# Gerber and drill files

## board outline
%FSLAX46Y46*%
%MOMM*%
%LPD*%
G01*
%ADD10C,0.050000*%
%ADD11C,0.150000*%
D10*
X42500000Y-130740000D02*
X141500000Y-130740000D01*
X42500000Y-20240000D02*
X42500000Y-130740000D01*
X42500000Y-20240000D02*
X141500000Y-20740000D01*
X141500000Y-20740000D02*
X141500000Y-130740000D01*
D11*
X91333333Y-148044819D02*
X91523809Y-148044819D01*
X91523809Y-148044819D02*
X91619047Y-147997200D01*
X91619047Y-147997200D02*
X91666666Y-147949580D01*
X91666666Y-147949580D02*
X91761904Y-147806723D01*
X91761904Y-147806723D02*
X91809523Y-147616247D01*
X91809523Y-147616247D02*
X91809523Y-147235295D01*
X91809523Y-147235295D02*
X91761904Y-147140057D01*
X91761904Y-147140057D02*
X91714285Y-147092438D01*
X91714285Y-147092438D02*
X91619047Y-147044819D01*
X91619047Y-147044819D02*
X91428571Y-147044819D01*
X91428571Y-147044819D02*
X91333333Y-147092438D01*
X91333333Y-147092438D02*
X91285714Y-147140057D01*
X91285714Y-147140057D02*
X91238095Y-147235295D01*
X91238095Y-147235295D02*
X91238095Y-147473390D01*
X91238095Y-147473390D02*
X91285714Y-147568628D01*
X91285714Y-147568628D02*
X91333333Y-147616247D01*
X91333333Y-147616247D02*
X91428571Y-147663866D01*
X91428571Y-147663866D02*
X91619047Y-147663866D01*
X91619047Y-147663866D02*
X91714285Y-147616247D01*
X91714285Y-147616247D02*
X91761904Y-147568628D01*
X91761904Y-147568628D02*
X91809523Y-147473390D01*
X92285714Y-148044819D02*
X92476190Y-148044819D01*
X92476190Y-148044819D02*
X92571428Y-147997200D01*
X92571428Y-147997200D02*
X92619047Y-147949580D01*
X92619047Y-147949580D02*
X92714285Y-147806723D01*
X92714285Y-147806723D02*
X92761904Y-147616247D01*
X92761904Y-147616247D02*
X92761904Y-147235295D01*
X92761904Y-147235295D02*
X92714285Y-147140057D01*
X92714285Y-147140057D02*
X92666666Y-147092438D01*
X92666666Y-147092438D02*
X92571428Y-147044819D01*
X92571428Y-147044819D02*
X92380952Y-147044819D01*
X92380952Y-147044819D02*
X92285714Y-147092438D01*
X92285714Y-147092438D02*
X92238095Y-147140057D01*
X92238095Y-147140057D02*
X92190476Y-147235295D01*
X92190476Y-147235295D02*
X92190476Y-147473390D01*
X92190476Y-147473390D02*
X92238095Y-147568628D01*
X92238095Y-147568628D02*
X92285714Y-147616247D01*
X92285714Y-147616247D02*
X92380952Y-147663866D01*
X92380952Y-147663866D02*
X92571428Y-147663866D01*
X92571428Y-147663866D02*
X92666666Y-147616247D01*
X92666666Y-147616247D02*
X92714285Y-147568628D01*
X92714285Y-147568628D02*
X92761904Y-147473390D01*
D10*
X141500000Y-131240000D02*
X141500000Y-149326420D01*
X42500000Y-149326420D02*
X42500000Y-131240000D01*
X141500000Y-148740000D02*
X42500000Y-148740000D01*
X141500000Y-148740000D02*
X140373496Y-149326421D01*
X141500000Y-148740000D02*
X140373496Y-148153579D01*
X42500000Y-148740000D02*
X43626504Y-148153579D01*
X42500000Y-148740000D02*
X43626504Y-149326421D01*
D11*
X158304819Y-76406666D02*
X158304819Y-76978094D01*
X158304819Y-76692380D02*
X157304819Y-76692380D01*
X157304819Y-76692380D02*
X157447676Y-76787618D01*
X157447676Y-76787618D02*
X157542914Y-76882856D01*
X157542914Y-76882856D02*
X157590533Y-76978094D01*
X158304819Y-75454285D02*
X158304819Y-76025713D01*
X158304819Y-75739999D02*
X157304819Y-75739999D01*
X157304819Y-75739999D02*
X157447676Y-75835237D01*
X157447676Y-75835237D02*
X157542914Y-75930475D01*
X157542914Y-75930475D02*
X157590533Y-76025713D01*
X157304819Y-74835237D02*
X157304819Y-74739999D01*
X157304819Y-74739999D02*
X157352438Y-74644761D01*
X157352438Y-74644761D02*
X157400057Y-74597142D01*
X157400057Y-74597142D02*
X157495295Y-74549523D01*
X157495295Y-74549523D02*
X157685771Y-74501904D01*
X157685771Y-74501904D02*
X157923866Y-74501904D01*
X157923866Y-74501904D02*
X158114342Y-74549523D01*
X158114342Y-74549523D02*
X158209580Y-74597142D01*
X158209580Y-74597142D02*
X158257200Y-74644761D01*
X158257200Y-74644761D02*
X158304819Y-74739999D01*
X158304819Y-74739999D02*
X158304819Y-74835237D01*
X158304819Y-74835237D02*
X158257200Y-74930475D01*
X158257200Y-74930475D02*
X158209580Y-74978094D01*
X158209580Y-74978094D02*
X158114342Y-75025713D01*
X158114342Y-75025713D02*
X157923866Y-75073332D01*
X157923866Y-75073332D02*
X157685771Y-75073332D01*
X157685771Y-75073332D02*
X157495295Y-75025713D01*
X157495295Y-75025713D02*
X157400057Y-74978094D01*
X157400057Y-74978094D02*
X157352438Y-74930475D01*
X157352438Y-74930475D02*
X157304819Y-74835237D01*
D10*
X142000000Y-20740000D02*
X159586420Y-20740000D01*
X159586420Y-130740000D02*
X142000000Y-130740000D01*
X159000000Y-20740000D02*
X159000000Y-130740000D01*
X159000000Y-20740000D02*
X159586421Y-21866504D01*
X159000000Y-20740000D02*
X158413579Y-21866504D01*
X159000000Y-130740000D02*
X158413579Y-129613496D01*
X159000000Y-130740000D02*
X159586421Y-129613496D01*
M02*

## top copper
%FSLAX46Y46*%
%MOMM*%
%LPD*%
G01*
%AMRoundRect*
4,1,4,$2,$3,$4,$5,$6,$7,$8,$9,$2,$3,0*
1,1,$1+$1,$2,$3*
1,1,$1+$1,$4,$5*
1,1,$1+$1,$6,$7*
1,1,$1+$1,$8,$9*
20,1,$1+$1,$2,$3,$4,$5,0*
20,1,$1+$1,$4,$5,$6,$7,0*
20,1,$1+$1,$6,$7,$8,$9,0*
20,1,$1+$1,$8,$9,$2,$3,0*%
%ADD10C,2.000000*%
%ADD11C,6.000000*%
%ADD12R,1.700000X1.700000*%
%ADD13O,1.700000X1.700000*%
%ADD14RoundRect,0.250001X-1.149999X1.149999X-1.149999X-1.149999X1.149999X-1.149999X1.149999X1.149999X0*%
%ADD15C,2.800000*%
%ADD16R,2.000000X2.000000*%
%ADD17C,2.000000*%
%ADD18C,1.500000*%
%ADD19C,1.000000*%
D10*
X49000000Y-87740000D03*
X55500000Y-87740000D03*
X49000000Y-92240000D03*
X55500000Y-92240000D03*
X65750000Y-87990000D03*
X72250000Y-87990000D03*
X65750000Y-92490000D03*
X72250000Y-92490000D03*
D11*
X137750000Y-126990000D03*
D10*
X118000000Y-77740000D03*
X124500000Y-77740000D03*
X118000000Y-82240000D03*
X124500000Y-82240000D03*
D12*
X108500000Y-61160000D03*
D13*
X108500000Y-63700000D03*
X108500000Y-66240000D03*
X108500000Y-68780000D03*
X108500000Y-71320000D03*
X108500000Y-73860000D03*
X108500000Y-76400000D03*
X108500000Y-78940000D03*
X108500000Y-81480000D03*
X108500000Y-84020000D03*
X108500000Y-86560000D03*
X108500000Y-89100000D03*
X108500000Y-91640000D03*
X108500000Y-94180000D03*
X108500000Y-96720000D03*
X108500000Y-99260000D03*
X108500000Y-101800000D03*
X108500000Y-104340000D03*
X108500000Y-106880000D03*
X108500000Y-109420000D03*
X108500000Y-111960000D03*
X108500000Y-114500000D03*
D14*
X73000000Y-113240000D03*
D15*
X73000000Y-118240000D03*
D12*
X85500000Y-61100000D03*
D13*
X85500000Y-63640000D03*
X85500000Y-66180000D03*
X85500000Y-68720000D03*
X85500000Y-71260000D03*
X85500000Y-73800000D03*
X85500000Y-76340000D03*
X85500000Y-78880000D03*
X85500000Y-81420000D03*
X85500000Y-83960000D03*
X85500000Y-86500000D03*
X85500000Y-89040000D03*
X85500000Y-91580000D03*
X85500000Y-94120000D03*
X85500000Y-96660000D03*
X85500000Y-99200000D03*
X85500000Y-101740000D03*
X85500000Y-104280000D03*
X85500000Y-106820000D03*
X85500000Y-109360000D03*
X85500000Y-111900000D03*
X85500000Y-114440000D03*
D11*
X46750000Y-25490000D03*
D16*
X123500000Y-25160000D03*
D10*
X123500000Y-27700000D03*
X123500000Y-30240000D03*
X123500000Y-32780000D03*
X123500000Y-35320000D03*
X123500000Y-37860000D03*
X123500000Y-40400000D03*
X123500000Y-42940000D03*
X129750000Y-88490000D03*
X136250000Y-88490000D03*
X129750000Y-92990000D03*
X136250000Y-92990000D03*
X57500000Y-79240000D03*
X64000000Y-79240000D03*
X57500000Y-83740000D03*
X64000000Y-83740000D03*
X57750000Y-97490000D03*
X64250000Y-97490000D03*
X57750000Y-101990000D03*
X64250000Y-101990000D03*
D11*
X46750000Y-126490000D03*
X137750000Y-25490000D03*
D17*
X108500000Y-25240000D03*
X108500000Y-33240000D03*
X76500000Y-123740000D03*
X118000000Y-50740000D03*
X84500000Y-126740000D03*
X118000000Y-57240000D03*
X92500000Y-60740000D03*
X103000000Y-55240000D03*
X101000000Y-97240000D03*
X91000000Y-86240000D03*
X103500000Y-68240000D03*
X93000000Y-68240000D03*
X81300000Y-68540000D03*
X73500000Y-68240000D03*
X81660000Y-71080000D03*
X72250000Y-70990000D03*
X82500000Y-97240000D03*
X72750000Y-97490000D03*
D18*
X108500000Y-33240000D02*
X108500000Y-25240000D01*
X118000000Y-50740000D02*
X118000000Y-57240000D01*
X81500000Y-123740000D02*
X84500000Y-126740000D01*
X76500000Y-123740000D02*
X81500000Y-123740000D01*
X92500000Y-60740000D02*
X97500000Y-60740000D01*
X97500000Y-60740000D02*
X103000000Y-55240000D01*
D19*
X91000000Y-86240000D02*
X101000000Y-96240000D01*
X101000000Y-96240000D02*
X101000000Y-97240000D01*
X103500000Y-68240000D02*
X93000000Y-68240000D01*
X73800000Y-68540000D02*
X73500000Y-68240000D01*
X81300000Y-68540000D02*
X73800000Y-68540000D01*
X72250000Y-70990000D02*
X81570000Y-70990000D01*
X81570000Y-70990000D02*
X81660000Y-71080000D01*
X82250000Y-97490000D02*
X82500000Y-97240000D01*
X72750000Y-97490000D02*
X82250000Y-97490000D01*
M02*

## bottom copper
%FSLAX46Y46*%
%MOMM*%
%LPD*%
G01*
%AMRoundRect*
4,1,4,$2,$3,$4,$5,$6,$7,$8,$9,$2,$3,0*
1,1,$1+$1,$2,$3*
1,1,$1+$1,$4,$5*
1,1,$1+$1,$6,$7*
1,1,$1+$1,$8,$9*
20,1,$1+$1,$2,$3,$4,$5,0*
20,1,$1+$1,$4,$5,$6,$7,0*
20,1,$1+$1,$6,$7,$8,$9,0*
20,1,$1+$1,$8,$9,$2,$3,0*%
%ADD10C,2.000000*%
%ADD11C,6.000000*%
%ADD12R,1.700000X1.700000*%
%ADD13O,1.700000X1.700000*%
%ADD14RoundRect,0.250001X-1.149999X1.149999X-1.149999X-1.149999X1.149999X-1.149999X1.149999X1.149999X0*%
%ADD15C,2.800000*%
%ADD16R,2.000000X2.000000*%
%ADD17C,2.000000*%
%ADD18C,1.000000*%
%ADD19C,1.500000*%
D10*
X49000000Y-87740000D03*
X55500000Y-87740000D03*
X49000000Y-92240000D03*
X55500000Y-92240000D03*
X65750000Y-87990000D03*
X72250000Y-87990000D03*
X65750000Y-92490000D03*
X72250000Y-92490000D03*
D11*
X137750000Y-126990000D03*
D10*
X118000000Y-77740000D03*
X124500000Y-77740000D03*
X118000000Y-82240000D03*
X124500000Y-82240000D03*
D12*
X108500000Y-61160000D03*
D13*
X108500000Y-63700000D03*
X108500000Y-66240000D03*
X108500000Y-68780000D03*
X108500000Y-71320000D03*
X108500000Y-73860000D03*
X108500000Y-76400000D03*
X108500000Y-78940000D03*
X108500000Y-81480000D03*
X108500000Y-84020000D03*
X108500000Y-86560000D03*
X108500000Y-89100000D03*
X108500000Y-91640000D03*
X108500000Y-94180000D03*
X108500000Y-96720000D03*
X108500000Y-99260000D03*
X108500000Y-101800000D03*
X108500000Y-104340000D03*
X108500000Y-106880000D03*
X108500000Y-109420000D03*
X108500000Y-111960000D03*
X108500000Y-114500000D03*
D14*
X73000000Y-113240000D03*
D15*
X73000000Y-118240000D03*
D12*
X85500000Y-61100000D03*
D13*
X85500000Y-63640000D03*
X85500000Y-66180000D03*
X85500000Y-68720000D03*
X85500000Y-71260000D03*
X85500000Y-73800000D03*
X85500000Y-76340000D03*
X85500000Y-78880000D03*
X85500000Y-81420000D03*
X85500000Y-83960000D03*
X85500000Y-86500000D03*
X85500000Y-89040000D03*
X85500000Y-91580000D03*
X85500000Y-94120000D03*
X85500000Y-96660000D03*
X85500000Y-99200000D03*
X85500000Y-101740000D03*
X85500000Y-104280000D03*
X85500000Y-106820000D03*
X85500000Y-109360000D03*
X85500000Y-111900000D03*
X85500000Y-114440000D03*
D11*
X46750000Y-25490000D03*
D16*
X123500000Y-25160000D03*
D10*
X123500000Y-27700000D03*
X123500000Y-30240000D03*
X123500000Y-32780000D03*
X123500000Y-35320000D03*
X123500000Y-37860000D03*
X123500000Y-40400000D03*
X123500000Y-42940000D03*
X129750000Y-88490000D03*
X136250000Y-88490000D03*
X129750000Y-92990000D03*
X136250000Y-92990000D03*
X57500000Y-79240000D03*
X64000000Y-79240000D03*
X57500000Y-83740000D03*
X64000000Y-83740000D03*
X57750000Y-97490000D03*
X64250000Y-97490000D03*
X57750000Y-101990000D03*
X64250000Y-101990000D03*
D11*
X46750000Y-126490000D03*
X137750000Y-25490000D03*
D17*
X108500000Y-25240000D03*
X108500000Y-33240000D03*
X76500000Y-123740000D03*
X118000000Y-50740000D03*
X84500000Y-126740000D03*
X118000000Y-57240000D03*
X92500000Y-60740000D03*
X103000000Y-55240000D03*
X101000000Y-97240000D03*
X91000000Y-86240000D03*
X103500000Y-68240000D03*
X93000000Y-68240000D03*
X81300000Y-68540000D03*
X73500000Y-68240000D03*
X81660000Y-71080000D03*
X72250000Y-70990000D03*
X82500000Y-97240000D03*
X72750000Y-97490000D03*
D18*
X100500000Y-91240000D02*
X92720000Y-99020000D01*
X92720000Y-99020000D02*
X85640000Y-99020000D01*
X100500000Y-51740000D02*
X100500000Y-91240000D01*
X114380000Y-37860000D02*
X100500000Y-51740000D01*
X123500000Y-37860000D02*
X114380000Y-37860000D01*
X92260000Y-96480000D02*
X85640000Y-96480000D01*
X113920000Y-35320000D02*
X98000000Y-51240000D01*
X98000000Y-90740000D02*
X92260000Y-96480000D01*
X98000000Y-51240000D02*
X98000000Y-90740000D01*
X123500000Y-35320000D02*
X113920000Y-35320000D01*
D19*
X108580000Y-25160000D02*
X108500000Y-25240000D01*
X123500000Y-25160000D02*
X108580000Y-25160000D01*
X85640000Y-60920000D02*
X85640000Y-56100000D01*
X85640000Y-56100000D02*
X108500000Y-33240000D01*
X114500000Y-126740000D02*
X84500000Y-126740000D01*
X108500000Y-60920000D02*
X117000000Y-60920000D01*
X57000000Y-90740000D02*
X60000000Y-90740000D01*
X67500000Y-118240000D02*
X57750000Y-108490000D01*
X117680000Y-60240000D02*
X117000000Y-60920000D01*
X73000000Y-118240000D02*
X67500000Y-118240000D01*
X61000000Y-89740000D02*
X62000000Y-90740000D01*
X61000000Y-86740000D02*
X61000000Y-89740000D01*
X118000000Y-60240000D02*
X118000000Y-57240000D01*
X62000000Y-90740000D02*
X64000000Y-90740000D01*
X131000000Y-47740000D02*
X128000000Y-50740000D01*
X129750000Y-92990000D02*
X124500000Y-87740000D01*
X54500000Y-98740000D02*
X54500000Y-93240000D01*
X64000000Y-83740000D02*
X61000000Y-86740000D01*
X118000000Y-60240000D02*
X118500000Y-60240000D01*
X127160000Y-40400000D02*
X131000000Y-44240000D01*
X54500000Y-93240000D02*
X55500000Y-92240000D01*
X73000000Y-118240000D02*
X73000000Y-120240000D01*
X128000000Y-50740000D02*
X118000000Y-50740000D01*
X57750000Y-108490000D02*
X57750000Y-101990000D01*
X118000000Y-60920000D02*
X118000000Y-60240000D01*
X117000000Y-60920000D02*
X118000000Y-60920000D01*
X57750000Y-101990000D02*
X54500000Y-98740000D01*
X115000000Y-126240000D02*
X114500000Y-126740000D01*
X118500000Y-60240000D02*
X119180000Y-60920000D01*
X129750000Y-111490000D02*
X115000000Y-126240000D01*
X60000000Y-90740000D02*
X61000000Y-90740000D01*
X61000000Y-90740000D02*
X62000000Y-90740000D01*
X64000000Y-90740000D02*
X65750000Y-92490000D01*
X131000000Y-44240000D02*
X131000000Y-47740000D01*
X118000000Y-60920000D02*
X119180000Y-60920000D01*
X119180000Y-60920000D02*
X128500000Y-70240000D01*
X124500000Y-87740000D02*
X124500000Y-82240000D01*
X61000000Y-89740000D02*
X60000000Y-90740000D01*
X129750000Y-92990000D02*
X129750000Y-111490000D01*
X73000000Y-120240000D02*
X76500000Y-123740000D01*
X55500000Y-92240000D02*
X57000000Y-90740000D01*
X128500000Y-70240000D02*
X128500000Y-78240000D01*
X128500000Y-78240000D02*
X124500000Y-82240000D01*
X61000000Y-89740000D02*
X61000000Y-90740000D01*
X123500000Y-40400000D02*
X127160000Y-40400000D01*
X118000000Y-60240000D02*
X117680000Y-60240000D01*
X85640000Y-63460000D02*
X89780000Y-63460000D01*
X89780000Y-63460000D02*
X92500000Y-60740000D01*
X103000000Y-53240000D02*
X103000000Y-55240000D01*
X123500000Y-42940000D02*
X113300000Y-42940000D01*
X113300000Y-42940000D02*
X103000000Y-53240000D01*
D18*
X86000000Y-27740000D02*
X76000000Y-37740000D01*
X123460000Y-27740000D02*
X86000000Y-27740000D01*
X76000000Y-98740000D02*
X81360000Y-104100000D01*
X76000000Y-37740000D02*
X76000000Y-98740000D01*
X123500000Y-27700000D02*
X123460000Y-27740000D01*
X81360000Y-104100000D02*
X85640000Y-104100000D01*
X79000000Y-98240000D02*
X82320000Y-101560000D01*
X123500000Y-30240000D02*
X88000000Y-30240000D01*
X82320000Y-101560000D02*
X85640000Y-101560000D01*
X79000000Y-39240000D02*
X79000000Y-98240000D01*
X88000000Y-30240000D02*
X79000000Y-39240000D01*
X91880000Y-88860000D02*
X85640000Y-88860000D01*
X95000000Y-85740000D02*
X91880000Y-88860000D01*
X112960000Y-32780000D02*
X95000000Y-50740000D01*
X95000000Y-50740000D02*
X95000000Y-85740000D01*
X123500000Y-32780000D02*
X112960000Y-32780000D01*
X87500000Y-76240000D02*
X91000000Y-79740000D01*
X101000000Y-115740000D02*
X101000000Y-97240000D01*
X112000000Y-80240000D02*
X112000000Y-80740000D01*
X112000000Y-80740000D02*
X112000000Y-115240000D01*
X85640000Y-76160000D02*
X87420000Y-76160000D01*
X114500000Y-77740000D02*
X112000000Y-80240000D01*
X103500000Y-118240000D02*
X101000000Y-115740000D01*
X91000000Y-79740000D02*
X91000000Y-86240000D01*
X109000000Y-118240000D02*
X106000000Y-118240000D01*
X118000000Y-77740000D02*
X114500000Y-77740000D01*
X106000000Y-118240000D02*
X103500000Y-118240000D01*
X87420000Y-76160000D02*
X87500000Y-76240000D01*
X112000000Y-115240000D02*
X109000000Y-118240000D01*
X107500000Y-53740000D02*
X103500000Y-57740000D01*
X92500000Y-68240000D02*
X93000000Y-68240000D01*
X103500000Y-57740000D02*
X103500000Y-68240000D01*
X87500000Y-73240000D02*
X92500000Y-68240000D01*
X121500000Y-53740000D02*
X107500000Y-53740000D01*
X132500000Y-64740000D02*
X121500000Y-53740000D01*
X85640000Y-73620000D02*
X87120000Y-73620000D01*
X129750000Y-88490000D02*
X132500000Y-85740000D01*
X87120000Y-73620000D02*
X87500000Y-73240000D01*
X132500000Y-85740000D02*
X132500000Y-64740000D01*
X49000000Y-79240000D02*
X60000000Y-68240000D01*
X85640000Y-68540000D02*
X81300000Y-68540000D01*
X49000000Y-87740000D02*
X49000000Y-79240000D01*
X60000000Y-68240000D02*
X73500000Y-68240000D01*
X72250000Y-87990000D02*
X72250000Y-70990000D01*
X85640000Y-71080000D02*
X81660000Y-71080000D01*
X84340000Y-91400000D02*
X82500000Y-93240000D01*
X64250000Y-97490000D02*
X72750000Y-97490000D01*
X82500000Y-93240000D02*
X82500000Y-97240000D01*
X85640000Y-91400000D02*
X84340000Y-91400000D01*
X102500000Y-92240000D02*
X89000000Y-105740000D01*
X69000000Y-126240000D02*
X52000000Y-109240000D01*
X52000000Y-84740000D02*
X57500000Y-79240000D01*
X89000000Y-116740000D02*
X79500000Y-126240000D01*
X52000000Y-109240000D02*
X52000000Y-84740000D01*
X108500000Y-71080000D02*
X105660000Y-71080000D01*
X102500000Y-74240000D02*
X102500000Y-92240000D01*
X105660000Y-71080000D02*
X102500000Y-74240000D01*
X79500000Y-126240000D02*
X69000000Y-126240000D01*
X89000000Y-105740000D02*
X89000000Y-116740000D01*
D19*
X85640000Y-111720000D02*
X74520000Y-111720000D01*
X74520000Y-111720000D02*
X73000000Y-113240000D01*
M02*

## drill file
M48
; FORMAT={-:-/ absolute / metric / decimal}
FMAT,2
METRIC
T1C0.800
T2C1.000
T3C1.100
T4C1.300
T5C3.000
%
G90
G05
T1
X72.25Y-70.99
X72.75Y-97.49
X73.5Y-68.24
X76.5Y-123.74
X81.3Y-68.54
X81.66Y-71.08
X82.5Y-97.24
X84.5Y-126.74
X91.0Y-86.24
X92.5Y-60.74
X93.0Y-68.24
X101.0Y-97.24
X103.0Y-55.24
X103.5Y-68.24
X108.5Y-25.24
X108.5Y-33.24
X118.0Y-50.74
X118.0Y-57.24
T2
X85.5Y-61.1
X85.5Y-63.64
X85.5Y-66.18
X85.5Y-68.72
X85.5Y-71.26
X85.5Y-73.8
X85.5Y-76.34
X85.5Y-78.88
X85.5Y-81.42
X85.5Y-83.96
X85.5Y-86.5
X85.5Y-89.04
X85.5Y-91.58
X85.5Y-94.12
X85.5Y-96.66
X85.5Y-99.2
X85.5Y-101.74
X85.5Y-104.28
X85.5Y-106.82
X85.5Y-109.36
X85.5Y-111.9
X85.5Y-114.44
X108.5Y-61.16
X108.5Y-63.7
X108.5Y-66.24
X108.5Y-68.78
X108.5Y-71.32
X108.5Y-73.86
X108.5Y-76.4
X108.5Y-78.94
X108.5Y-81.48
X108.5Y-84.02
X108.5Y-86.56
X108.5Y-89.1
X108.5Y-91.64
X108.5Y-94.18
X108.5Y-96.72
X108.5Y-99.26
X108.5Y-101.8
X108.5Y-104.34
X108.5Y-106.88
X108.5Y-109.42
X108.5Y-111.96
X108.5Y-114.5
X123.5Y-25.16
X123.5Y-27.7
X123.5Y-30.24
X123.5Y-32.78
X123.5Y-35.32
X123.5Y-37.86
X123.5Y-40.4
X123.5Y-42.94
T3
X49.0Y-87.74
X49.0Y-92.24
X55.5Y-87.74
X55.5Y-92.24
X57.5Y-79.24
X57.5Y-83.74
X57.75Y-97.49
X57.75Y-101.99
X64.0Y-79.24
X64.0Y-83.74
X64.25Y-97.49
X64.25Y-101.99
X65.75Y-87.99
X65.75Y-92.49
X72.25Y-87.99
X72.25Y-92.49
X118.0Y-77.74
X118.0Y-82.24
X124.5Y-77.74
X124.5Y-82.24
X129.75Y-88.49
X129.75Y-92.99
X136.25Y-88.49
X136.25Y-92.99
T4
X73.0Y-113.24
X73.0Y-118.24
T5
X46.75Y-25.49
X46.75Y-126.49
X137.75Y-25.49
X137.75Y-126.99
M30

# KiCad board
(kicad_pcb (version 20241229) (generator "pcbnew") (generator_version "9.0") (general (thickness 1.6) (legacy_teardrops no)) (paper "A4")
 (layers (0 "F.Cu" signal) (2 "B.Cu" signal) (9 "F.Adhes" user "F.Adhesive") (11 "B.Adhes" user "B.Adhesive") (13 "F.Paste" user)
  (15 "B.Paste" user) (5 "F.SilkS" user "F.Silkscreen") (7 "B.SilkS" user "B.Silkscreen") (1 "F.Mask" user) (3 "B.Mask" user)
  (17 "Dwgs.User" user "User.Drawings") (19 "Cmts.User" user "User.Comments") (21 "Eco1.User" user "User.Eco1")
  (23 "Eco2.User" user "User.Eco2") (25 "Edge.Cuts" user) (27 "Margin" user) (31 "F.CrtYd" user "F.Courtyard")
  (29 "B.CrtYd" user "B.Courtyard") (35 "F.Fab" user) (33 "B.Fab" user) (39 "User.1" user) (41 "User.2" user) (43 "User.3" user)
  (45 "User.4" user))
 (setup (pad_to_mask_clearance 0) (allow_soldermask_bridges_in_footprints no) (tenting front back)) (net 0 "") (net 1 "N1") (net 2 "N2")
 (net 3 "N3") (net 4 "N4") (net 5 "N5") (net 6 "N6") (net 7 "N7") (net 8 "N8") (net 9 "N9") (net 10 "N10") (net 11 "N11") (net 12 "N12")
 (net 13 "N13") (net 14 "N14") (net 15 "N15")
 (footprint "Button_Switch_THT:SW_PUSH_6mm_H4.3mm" (layer "F.Cu") (at 49 87.74)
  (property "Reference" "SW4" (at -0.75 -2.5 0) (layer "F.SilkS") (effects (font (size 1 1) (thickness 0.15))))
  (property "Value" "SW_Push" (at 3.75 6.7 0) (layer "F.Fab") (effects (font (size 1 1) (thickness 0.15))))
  (pad "1" thru_hole circle (at 0 0 90) (size 2 2) (drill 1.1) (layers "*.Cu" "*.Mask") (remove_unused_layers no) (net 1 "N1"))
  (pad "1" thru_hole circle (at 6.5 0 90) (size 2 2) (drill 1.1) (layers "*.Cu" "*.Mask") (remove_unused_layers no) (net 1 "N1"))
  (pad "2" thru_hole circle (at 0 4.5 90) (size 2 2) (drill 1.1) (layers "*.Cu" "*.Mask") (remove_unused_layers no) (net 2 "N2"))
  (pad "2" thru_hole circle (at 6.5 4.5 90) (size 2 2) (drill 1.1) (layers "*.Cu" "*.Mask") (remove_unused_layers no) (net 2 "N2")))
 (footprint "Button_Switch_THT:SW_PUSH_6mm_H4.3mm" (layer "F.Cu") (at 65.75 87.99)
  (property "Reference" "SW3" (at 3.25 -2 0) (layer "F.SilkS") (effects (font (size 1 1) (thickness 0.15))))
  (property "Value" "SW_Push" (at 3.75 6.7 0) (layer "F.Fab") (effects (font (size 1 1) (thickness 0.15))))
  (pad "1" thru_hole circle (at 0 0 90) (size 2 2) (drill 1.1) (layers "*.Cu" "*.Mask") (remove_unused_layers no) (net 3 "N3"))
  (pad "1" thru_hole circle (at 6.5 0 90) (size 2 2) (drill 1.1) (layers "*.Cu" "*.Mask") (remove_unused_layers no) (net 3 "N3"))
  (pad "2" thru_hole circle (at 0 4.5 90) (size 2 2) (drill 1.1) (layers "*.Cu" "*.Mask") (remove_unused_layers no) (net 2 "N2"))
  (pad "2" thru_hole circle (at 6.5 4.5 90) (size 2 2) (drill 1.1) (layers "*.Cu" "*.Mask") (remove_unused_layers no) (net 2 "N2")))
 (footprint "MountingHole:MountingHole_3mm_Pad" (layer "F.Cu") (at 137.75 126.99)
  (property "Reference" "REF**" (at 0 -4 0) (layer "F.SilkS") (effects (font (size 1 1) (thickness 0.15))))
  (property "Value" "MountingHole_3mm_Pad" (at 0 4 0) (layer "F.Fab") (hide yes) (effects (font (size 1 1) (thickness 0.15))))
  (pad "1" thru_hole circle (at 0 0) (size 6 6) (drill 3) (layers "*.Cu" "*.Mask") (remove_unused_layers no)))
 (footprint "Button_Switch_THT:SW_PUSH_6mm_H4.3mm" (layer "F.Cu") (at 118 77.74)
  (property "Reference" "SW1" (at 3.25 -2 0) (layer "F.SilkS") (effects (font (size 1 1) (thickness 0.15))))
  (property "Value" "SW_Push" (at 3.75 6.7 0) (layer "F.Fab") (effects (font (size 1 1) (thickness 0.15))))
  (pad "1" thru_hole circle (at 0 0 90) (size 2 2) (drill 1.1) (layers "*.Cu" "*.Mask") (remove_unused_layers no) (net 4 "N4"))
  (pad "1" thru_hole circle (at 6.5 0 90) (size 2 2) (drill 1.1) (layers "*.Cu" "*.Mask") (remove_unused_layers no) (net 4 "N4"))
  (pad "2" thru_hole circle (at 0 4.5 90) (size 2 2) (drill 1.1) (layers "*.Cu" "*.Mask") (remove_unused_layers no) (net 2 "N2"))
  (pad "2" thru_hole circle (at 6.5 4.5 90) (size 2 2) (drill 1.1) (layers "*.Cu" "*.Mask") (remove_unused_layers no) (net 2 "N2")))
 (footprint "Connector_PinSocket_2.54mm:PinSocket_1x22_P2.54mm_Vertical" (layer "F.Cu") (at 108.5 61.16)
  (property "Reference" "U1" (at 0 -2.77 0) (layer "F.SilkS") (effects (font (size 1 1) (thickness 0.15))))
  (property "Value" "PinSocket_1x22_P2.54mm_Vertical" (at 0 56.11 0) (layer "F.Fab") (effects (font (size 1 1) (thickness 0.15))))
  (pad "1" thru_hole rect (at 0 0) (size 1.7 1.7) (drill 1) (layers "*.Cu" "*.Mask") (remove_unused_layers no))
  (pad "2" thru_hole oval (at 0 2.54) (size 1.7 1.7) (drill 1) (layers "*.Cu" "*.Mask") (remove_unused_layers no))
  (pad "3" thru_hole oval (at 0 5.08) (size 1.7 1.7) (drill 1) (layers "*.Cu" "*.Mask") (remove_unused_layers no))
  (pad "4" thru_hole oval (at 0 7.62) (size 1.7 1.7) (drill 1) (layers "*.Cu" "*.Mask") (remove_unused_layers no))
  (pad "5" thru_hole oval (at 0 10.16) (size 1.7 1.7) (drill 1) (layers "*.Cu" "*.Mask") (remove_unused_layers no))
  (pad "6" thru_hole oval (at 0 12.7) (size 1.7 1.7) (drill 1) (layers "*.Cu" "*.Mask") (remove_unused_layers no))
  (pad "7" thru_hole oval (at 0 15.24) (size 1.7 1.7) (drill 1) (layers "*.Cu" "*.Mask") (remove_unused_layers no))
  (pad "8" thru_hole oval (at 0 17.78) (size 1.7 1.7) (drill 1) (layers "*.Cu" "*.Mask") (remove_unused_layers no))
  (pad "9" thru_hole oval (at 0 20.32) (size 1.7 1.7) (drill 1) (layers "*.Cu" "*.Mask") (remove_unused_layers no))
  (pad "10" thru_hole oval (at 0 22.86) (size 1.7 1.7) (drill 1) (layers "*.Cu" "*.Mask") (remove_unused_layers no))
  (pad "11" thru_hole oval (at 0 25.4) (size 1.7 1.7) (drill 1) (layers "*.Cu" "*.Mask") (remove_unused_layers no))
  (pad "12" thru_hole oval (at 0 27.94) (size 1.7 1.7) (drill 1) (layers "*.Cu" "*.Mask") (remove_unused_layers no))
  (pad "13" thru_hole oval (at 0 30.48) (size 1.7 1.7) (drill 1) (layers "*.Cu" "*.Mask") (remove_unused_layers no))
  (pad "14" thru_hole oval (at 0 33.02) (size 1.7 1.7) (drill 1) (layers "*.Cu" "*.Mask") (remove_unused_layers no))
  (pad "15" thru_hole oval (at 0 35.56) (size 1.7 1.7) (drill 1) (layers "*.Cu" "*.Mask") (remove_unused_layers no))
  (pad "16" thru_hole oval (at 0 38.1) (size 1.7 1.7) (drill 1) (layers "*.Cu" "*.Mask") (remove_unused_layers no))
  (pad "17" thru_hole oval (at 0 40.64) (size 1.7 1.7) (drill 1) (layers "*.Cu" "*.Mask") (remove_unused_layers no))
  (pad "18" thru_hole oval (at 0 43.18) (size 1.7 1.7) (drill 1) (layers "*.Cu" "*.Mask") (remove_unused_layers no))
  (pad "19" thru_hole oval (at 0 45.72) (size 1.7 1.7) (drill 1) (layers "*.Cu" "*.Mask") (remove_unused_layers no))
  (pad "20" thru_hole oval (at 0 48.26) (size 1.7 1.7) (drill 1) (layers "*.Cu" "*.Mask") (remove_unused_layers no))
  (pad "21" thru_hole oval (at 0 50.8) (size 1.7 1.7) (drill 1) (layers "*.Cu" "*.Mask") (remove_unused_layers no))
  (pad "22" thru_hole oval (at 0 53.34) (size 1.7 1.7) (drill 1) (layers "*.Cu" "*.Mask") (remove_unused_layers no)))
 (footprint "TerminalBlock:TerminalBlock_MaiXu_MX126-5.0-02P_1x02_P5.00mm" (layer "F.Cu") (at 73 113.24 -90)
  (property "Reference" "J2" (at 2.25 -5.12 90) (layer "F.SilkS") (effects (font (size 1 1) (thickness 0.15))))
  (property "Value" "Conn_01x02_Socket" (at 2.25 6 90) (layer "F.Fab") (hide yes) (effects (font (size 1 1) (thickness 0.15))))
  (pad "1" thru_hole roundrect (at 0 0 270) (size 2.8 2.8) (drill 1.3) (layers "*.Cu" "*.Mask") (remove_unused_layers no)
   (roundrect_rratio 0.089286) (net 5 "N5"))
  (pad "2" thru_hole circle (at 5 0 270) (size 2.8 2.8) (drill 1.3) (layers "*.Cu" "*.Mask") (remove_unused_layers no) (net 2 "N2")))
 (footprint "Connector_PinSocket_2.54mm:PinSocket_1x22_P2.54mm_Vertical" (layer "F.Cu") (at 85.5 61.1)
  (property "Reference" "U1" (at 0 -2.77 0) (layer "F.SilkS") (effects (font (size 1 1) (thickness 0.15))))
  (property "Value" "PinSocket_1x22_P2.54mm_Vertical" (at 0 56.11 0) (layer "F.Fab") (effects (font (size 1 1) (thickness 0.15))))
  (pad "1" thru_hole rect (at 0 0) (size 1.7 1.7) (drill 1) (layers "*.Cu" "*.Mask") (remove_unused_layers no))
  (pad "2" thru_hole oval (at 0 2.54) (size 1.7 1.7) (drill 1) (layers "*.Cu" "*.Mask") (remove_unused_layers no))
  (pad "3" thru_hole oval (at 0 5.08) (size 1.7 1.7) (drill 1) (layers "*.Cu" "*.Mask") (remove_unused_layers no))
  (pad "4" thru_hole oval (at 0 7.62) (size 1.7 1.7) (drill 1) (layers "*.Cu" "*.Mask") (remove_unused_layers no))
  (pad "5" thru_hole oval (at 0 10.16) (size 1.7 1.7) (drill 1) (layers "*.Cu" "*.Mask") (remove_unused_layers no))
  (pad "6" thru_hole oval (at 0 12.7) (size 1.7 1.7) (drill 1) (layers "*.Cu" "*.Mask") (remove_unused_layers no))
  (pad "7" thru_hole oval (at 0 15.24) (size 1.7 1.7) (drill 1) (layers "*.Cu" "*.Mask") (remove_unused_layers no))
  (pad "8" thru_hole oval (at 0 17.78) (size 1.7 1.7) (drill 1) (layers "*.Cu" "*.Mask") (remove_unused_layers no))
  (pad "9" thru_hole oval (at 0 20.32) (size 1.7 1.7) (drill 1) (layers "*.Cu" "*.Mask") (remove_unused_layers no))
  (pad "10" thru_hole oval (at 0 22.86) (size 1.7 1.7) (drill 1) (layers "*.Cu" "*.Mask") (remove_unused_layers no))
  (pad "11" thru_hole oval (at 0 25.4) (size 1.7 1.7) (drill 1) (layers "*.Cu" "*.Mask") (remove_unused_layers no))
  (pad "12" thru_hole oval (at 0 27.94) (size 1.7 1.7) (drill 1) (layers "*.Cu" "*.Mask") (remove_unused_layers no))
  (pad "13" thru_hole oval (at 0 30.48) (size 1.7 1.7) (drill 1) (layers "*.Cu" "*.Mask") (remove_unused_layers no))
  (pad "14" thru_hole oval (at 0 33.02) (size 1.7 1.7) (drill 1) (layers "*.Cu" "*.Mask") (remove_unused_layers no))
  (pad "15" thru_hole oval (at 0 35.56) (size 1.7 1.7) (drill 1) (layers "*.Cu" "*.Mask") (remove_unused_layers no))
  (pad "16" thru_hole oval (at 0 38.1) (size 1.7 1.7) (drill 1) (layers "*.Cu" "*.Mask") (remove_unused_layers no))
  (pad "17" thru_hole oval (at 0 40.64) (size 1.7 1.7) (drill 1) (layers "*.Cu" "*.Mask") (remove_unused_layers no))
  (pad "18" thru_hole oval (at 0 43.18) (size 1.7 1.7) (drill 1) (layers "*.Cu" "*.Mask") (remove_unused_layers no))
  (pad "19" thru_hole oval (at 0 45.72) (size 1.7 1.7) (drill 1) (layers "*.Cu" "*.Mask") (remove_unused_layers no))
  (pad "20" thru_hole oval (at 0 48.26) (size 1.7 1.7) (drill 1) (layers "*.Cu" "*.Mask") (remove_unused_layers no))
  (pad "21" thru_hole oval (at 0 50.8) (size 1.7 1.7) (drill 1) (layers "*.Cu" "*.Mask") (remove_unused_layers no))
  (pad "22" thru_hole oval (at 0 53.34) (size 1.7 1.7) (drill 1) (layers "*.Cu" "*.Mask") (remove_unused_layers no)))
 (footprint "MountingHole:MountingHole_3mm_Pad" (layer "F.Cu") (at 46.75 25.49)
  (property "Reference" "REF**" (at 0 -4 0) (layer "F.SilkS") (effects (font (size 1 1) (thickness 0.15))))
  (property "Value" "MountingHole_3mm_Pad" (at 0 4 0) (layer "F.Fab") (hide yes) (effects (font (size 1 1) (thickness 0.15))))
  (pad "1" thru_hole circle (at 0 0) (size 6 6) (drill 3) (layers "*.Cu" "*.Mask") (remove_unused_layers no)))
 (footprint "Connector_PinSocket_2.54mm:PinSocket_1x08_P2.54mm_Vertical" (layer "F.Cu") (at 123.5 25.16)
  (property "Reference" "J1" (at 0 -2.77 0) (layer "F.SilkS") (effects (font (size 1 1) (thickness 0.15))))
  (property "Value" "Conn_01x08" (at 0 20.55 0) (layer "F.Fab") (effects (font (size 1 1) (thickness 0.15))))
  (pad "1" thru_hole rect (at 0 0) (size 2 2) (drill 1) (layers "*.Cu" "*.Mask") (remove_unused_layers no) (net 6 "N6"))
  (pad "2" thru_hole circle (at 0 2.54) (size 2 2) (drill 1) (layers "*.Cu" "*.Mask") (remove_unused_layers no) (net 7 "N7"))
  (pad "3" thru_hole circle (at 0 5.08) (size 2 2) (drill 1) (layers "*.Cu" "*.Mask") (remove_unused_layers no) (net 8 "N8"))
  (pad "4" thru_hole circle (at 0 7.62) (size 2 2) (drill 1) (layers "*.Cu" "*.Mask") (remove_unused_layers no) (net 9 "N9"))
  (pad "5" thru_hole circle (at 0 10.16) (size 2 2) (drill 1) (layers "*.Cu" "*.Mask") (remove_unused_layers no) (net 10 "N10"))
  (pad "6" thru_hole circle (at 0 12.7) (size 2 2) (drill 1) (layers "*.Cu" "*.Mask") (remove_unused_layers no) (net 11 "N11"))
  (pad "7" thru_hole circle (at 0 15.24) (size 2 2) (drill 1) (layers "*.Cu" "*.Mask") (remove_unused_layers no) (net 2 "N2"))
  (pad "8" thru_hole circle (at 0 17.78) (size 2 2) (drill 1) (layers "*.Cu" "*.Mask") (remove_unused_layers no) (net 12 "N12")))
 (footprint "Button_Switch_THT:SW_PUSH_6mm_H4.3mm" (layer "F.Cu") (at 129.75 88.49)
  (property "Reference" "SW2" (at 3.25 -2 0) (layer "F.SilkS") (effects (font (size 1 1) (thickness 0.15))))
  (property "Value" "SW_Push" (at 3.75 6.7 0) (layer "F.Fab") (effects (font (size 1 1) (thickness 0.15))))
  (pad "1" thru_hole circle (at 0 0 90) (size 2 2) (drill 1.1) (layers "*.Cu" "*.Mask") (remove_unused_layers no) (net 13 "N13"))
  (pad "1" thru_hole circle (at 6.5 0 90) (size 2 2) (drill 1.1) (layers "*.Cu" "*.Mask") (remove_unused_layers no) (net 13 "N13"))
  (pad "2" thru_hole circle (at 0 4.5 90) (size 2 2) (drill 1.1) (layers "*.Cu" "*.Mask") (remove_unused_layers no) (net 2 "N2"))
  (pad "2" thru_hole circle (at 6.5 4.5 90) (size 2 2) (drill 1.1) (layers "*.Cu" "*.Mask") (remove_unused_layers no) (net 2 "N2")))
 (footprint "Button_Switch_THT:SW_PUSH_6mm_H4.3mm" (layer "F.Cu") (at 57.5 79.24)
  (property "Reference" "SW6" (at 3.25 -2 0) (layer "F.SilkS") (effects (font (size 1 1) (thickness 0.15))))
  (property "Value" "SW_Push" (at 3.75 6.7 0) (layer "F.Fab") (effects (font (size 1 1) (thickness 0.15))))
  (pad "1" thru_hole circle (at 0 0 90) (size 2 2) (drill 1.1) (layers "*.Cu" "*.Mask") (remove_unused_layers no) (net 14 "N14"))
  (pad "1" thru_hole circle (at 6.5 0 90) (size 2 2) (drill 1.1) (layers "*.Cu" "*.Mask") (remove_unused_layers no) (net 14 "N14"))
  (pad "2" thru_hole circle (at 0 4.5 90) (size 2 2) (drill 1.1) (layers "*.Cu" "*.Mask") (remove_unused_layers no) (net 2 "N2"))
  (pad "2" thru_hole circle (at 6.5 4.5 90) (size 2 2) (drill 1.1) (layers "*.Cu" "*.Mask") (remove_unused_layers no) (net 2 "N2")))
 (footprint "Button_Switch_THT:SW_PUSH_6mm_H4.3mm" (layer "F.Cu") (at 57.75 97.49)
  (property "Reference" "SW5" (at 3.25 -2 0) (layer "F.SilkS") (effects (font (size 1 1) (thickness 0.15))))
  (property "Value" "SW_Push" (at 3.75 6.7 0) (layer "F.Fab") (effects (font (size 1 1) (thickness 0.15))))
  (pad "1" thru_hole circle (at 0 0 90) (size 2 2) (drill 1.1) (layers "*.Cu" "*.Mask") (remove_unused_layers no) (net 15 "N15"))
  (pad "1" thru_hole circle (at 6.5 0 90) (size 2 2) (drill 1.1) (layers "*.Cu" "*.Mask") (remove_unused_layers no) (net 15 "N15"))
  (pad "2" thru_hole circle (at 0 4.5 90) (size 2 2) (drill 1.1) (layers "*.Cu" "*.Mask") (remove_unused_layers no) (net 2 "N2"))
  (pad "2" thru_hole circle (at 6.5 4.5 90) (size 2 2) (drill 1.1) (layers "*.Cu" "*.Mask") (remove_unused_layers no) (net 2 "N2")))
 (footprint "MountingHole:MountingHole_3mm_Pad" (layer "F.Cu") (at 46.75 126.49)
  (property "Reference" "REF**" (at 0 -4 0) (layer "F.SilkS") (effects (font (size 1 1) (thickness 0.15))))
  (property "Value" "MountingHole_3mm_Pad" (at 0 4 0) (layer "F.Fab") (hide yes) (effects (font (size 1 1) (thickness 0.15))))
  (pad "1" thru_hole circle (at 0 0) (size 6 6) (drill 3) (layers "*.Cu" "*.Mask") (remove_unused_layers no)))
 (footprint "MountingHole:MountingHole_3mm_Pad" (layer "F.Cu") (at 137.75 25.49)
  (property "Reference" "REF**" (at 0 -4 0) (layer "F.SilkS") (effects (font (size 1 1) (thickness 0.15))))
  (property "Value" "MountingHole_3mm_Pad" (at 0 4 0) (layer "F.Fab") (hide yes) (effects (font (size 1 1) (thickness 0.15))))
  (pad "1" thru_hole circle (at 0 0) (size 6 6) (drill 3) (layers "*.Cu" "*.Mask") (remove_unused_layers no)))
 (gr_line (start 42.5 130.74) (end 141.5 130.74) (stroke (width 0.05) (type default)) (layer "Edge.Cuts"))
 (gr_line (start 42.5 20.24) (end 42.5 130.74) (stroke (width 0.05) (type default)) (layer "Edge.Cuts"))
 (gr_line (start 42.5 20.24) (end 141.5 20.74) (stroke (width 0.05) (type default)) (layer "Edge.Cuts"))
 (gr_line (start 141.5 20.74) (end 141.5 130.74) (stroke (width 0.05) (type default)) (layer "Edge.Cuts"))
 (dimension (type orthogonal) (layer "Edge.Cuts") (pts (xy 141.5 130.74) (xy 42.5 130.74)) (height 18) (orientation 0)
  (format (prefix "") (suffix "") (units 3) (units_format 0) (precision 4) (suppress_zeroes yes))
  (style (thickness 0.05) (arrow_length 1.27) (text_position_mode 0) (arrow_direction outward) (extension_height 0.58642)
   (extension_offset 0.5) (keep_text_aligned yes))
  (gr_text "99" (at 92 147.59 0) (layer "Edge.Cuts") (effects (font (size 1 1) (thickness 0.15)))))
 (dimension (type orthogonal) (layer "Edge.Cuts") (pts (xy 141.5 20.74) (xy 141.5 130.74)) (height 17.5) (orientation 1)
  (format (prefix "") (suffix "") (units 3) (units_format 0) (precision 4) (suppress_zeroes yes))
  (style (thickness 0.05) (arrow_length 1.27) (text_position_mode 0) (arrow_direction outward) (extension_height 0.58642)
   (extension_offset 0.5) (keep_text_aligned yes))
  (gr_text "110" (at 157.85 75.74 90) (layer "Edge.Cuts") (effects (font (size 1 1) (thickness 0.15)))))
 (segment (start 100.5 91.24) (end 92.72 99.02) (width 1) (layer "B.Cu") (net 11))
 (segment (start 92.72 99.02) (end 85.64 99.02) (width 1) (layer "B.Cu") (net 11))
 (segment (start 100.5 51.74) (end 100.5 91.24) (width 1) (layer "B.Cu") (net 11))
 (segment (start 114.38 37.86) (end 100.5 51.74) (width 1) (layer "B.Cu") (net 11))
 (segment (start 123.5 37.86) (end 114.38 37.86) (width 1) (layer "B.Cu") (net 11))
 (segment (start 92.26 96.48) (end 85.64 96.48) (width 1) (layer "B.Cu") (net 10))
 (segment (start 113.92 35.32) (end 98 51.24) (width 1) (layer "B.Cu") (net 10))
 (segment (start 98 90.74) (end 92.26 96.48) (width 1) (layer "B.Cu") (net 10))
 (segment (start 98 51.24) (end 98 90.74) (width 1) (layer "B.Cu") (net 10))
 (segment (start 123.5 35.32) (end 113.92 35.32) (width 1) (layer "B.Cu") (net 10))
 (segment (start 108.5 33.24) (end 108.5 25.24) (width 1.5) (layer "F.Cu") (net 6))
 (via (at 108.5 25.24) (size 2) (drill 0.8) (layers "F.Cu" "B.Cu") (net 6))
 (via (at 108.5 33.24) (size 2) (drill 0.8) (layers "F.Cu" "B.Cu") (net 6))
 (segment (start 108.58 25.16) (end 108.5 25.24) (width 1.5) (layer "B.Cu") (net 6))
 (segment (start 123.5 25.16) (end 108.58 25.16) (width 1.5) (layer "B.Cu") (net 6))
 (segment (start 85.64 60.92) (end 85.64 56.1) (width 1.5) (layer "B.Cu") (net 6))
 (segment (start 85.64 56.1) (end 108.5 33.24) (width 1.5) (layer "B.Cu") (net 6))
 (segment (start 118 50.74) (end 118 57.24) (width 1.5) (layer "F.Cu") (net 2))
 (segment (start 81.5 123.74) (end 84.5 126.74) (width 1.5) (layer "F.Cu") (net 2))
 (segment (start 76.5 123.74) (end 81.5 123.74) (width 1.5) (layer "F.Cu") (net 2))
 (via (at 76.5 123.74) (size 2) (drill 0.8) (layers "F.Cu" "B.Cu") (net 2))
 (via (at 118 50.74) (size 2) (drill 0.8) (layers "F.Cu" "B.Cu") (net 2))
 (via (at 84.5 126.74) (size 2) (drill 0.8) (layers "F.Cu" "B.Cu") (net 2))
 (via (at 118 57.24) (size 2) (drill 0.8) (layers "F.Cu" "B.Cu") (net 2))
 (segment (start 114.5 126.74) (end 84.5 126.74) (width 1.5) (layer "B.Cu") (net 2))
 (segment (start 108.5 60.92) (end 117 60.92) (width 1.5) (layer "B.Cu") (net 2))
 (segment (start 57 90.74) (end 60 90.74) (width 1.5) (layer "B.Cu") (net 2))
 (segment (start 67.5 118.24) (end 57.75 108.49) (width 1.5) (layer "B.Cu") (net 2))
 (segment (start 117.68 60.24) (end 117 60.92) (width 1.5) (layer "B.Cu") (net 2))
 (segment (start 73 118.24) (end 67.5 118.24) (width 1.5) (layer "B.Cu") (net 2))
 (segment (start 61 89.74) (end 62 90.74) (width 1.5) (layer "B.Cu") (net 2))
 (segment (start 61 86.74) (end 61 89.74) (width 1.5) (layer "B.Cu") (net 2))
 (segment (start 118 60.24) (end 118 57.24) (width 1.5) (layer "B.Cu") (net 2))
 (segment (start 62 90.74) (end 64 90.74) (width 1.5) (layer "B.Cu") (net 2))
 (segment (start 131 47.74) (end 128 50.74) (width 1.5) (layer "B.Cu") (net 2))
 (segment (start 129.75 92.99) (end 124.5 87.74) (width 1.5) (layer "B.Cu") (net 2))
 (segment (start 54.5 98.74) (end 54.5 93.24) (width 1.5) (layer "B.Cu") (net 2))
 (segment (start 64 83.74) (end 61 86.74) (width 1.5) (layer "B.Cu") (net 2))
 (segment (start 118 60.24) (end 118.5 60.24) (width 1.5) (layer "B.Cu") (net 2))
 (segment (start 127.16 40.4) (end 131 44.24) (width 1.5) (layer "B.Cu") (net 2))
 (segment (start 54.5 93.24) (end 55.5 92.24) (width 1.5) (layer "B.Cu") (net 2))
 (segment (start 73 118.24) (end 73 120.24) (width 1.5) (layer "B.Cu") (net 2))
 (segment (start 128 50.74) (end 118 50.74) (width 1.5) (layer "B.Cu") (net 2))
 (segment (start 57.75 108.49) (end 57.75 101.99) (width 1.5) (layer "B.Cu") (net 2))
 (segment (start 118 60.92) (end 118 60.24) (width 1.5) (layer "B.Cu") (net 2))
 (segment (start 117 60.92) (end 118 60.92) (width 1.5) (layer "B.Cu") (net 2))
 (segment (start 57.75 101.99) (end 54.5 98.74) (width 1.5) (layer "B.Cu") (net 2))
 (segment (start 115 126.24) (end 114.5 126.74) (width 1.5) (layer "B.Cu") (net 2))
 (segment (start 118.5 60.24) (end 119.18 60.92) (width 1.5) (layer "B.Cu") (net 2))
 (segment (start 129.75 111.49) (end 115 126.24) (width 1.5) (layer "B.Cu") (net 2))
 (segment (start 60 90.74) (end 61 90.74) (width 1.5) (layer "B.Cu") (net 2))
 (segment (start 61 90.74) (end 62 90.74) (width 1.5) (layer "B.Cu") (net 2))
 (segment (start 64 90.74) (end 65.75 92.49) (width 1.5) (layer "B.Cu") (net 2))
 (segment (start 131 44.24) (end 131 47.74) (width 1.5) (layer "B.Cu") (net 2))
 (segment (start 118 60.92) (end 119.18 60.92) (width 1.5) (layer "B.Cu") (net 2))
 (segment (start 119.18 60.92) (end 128.5 70.24) (width 1.5) (layer "B.Cu") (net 2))
 (segment (start 124.5 87.74) (end 124.5 82.24) (width 1.5) (layer "B.Cu") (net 2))
 (segment (start 61 89.74) (end 60 90.74) (width 1.5) (layer "B.Cu") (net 2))
 (segment (start 129.75 92.99) (end 129.75 111.49) (width 1.5) (layer "B.Cu") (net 2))
 (segment (start 73 120.24) (end 76.5 123.74) (width 1.5) (layer "B.Cu") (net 2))
 (segment (start 55.5 92.24) (end 57 90.74) (width 1.5) (layer "B.Cu") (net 2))
 (segment (start 128.5 70.24) (end 128.5 78.24) (width 1.5) (layer "B.Cu") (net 2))
 (segment (start 128.5 78.24) (end 124.5 82.24) (width 1.5) (layer "B.Cu") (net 2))
 (segment (start 61 89.74) (end 61 90.74) (width 1.5) (layer "B.Cu") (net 2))
 (segment (start 123.5 40.4) (end 127.16 40.4) (width 1.5) (layer "B.Cu") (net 2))
 (segment (start 118 60.24) (end 117.68 60.24) (width 1.5) (layer "B.Cu") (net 2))
 (segment (start 92.5 60.74) (end 97.5 60.74) (width 1.5) (layer "F.Cu") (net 12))
 (segment (start 97.5 60.74) (end 103 55.24) (width 1.5) (layer "F.Cu") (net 12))
 (via (at 92.5 60.74) (size 2) (drill 0.8) (layers "F.Cu" "B.Cu") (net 12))
 (via (at 103 55.24) (size 2) (drill 0.8) (layers "F.Cu" "B.Cu") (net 12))
 (segment (start 85.64 63.46) (end 89.78 63.46) (width 1.5) (layer "B.Cu") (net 12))
 (segment (start 89.78 63.46) (end 92.5 60.74) (width 1.5) (layer "B.Cu") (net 12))
 (segment (start 103 53.24) (end 103 55.24) (width 1.5) (layer "B.Cu") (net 12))
 (segment (start 123.5 42.94) (end 113.3 42.94) (width 1.5) (layer "B.Cu") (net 12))
 (segment (start 113.3 42.94) (end 103 53.24) (width 1.5) (layer "B.Cu") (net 12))
 (segment (start 86 27.74) (end 76 37.74) (width 1) (layer "B.Cu") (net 7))
 (segment (start 123.46 27.74) (end 86 27.74) (width 1) (layer "B.Cu") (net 7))
 (segment (start 76 98.74) (end 81.36 104.1) (width 1) (layer "B.Cu") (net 7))
 (segment (start 76 37.74) (end 76 98.74) (width 1) (layer "B.Cu") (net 7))
 (segment (start 123.5 27.7) (end 123.46 27.74) (width 1) (layer "B.Cu") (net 7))
 (segment (start 81.36 104.1) (end 85.64 104.1) (width 1) (layer "B.Cu") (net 7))
 (segment (start 79 98.24) (end 82.32 101.56) (width 1) (layer "B.Cu") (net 8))
 (segment (start 123.5 30.24) (end 88 30.24) (width 1) (layer "B.Cu") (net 8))
 (segment (start 82.32 101.56) (end 85.64 101.56) (width 1) (layer "B.Cu") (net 8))
 (segment (start 79 39.24) (end 79 98.24) (width 1) (layer "B.Cu") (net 8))
 (segment (start 88 30.24) (end 79 39.24) (width 1) (layer "B.Cu") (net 8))
 (segment (start 91.88 88.86) (end 85.64 88.86) (width 1) (layer "B.Cu") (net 9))
 (segment (start 95 85.74) (end 91.88 88.86) (width 1) (layer "B.Cu") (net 9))
 (segment (start 112.96 32.78) (end 95 50.74) (width 1) (layer "B.Cu") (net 9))
 (segment (start 95 50.74) (end 95 85.74) (width 1) (layer "B.Cu") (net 9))
 (segment (start 123.5 32.78) (end 112.96 32.78) (width 1) (layer "B.Cu") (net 9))
 (segment (start 91 86.24) (end 101 96.24) (width 1) (layer "F.Cu") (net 4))
 (segment (start 101 96.24) (end 101 97.24) (width 1) (layer "F.Cu") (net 4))
 (via (at 101 97.24) (size 2) (drill 0.8) (layers "F.Cu" "B.Cu") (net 4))
 (via (at 91 86.24) (size 2) (drill 0.8) (layers "F.Cu" "B.Cu") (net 4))
 (segment (start 87.5 76.24) (end 91 79.74) (width 1) (layer "B.Cu") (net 4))
 (segment (start 101 115.74) (end 101 97.24) (width 1) (layer "B.Cu") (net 4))
 (segment (start 112 80.24) (end 112 80.74) (width 1) (layer "B.Cu") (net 4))
 (segment (start 112 80.74) (end 112 115.24) (width 1) (layer "B.Cu") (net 4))
 (segment (start 85.64 76.16) (end 87.42 76.16) (width 1) (layer "B.Cu") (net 4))
 (segment (start 114.5 77.74) (end 112 80.24) (width 1) (layer "B.Cu") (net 4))
 (segment (start 103.5 118.24) (end 101 115.74) (width 1) (layer "B.Cu") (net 4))
 (segment (start 91 79.74) (end 91 86.24) (width 1) (layer "B.Cu") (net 4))
 (segment (start 109 118.24) (end 106 118.24) (width 1) (layer "B.Cu") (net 4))
 (segment (start 118 77.74) (end 114.5 77.74) (width 1) (layer "B.Cu") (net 4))
 (segment (start 106 118.24) (end 103.5 118.24) (width 1) (layer "B.Cu") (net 4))
 (segment (start 87.42 76.16) (end 87.5 76.24) (width 1) (layer "B.Cu") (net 4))
 (segment (start 112 115.24) (end 109 118.24) (width 1) (layer "B.Cu") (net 4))
 (segment (start 103.5 68.24) (end 93 68.24) (width 1) (layer "F.Cu") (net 13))
 (via (at 103.5 68.24) (size 2) (drill 0.8) (layers "F.Cu" "B.Cu") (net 13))
 (via (at 93 68.24) (size 2) (drill 0.8) (layers "F.Cu" "B.Cu") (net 13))
 (segment (start 107.5 53.74) (end 103.5 57.74) (width 1) (layer "B.Cu") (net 13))
 (segment (start 92.5 68.24) (end 93 68.24) (width 1) (layer "B.Cu") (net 13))
 (segment (start 103.5 57.74) (end 103.5 68.24) (width 1) (layer "B.Cu") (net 13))
 (segment (start 87.5 73.24) (end 92.5 68.24) (width 1) (layer "B.Cu") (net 13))
 (segment (start 121.5 53.74) (end 107.5 53.74) (width 1) (layer "B.Cu") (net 13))
 (segment (start 132.5 64.74) (end 121.5 53.74) (width 1) (layer "B.Cu") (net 13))
 (segment (start 85.64 73.62) (end 87.12 73.62) (width 1) (layer "B.Cu") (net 13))
 (segment (start 129.75 88.49) (end 132.5 85.74) (width 1) (layer "B.Cu") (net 13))
 (segment (start 87.12 73.62) (end 87.5 73.24) (width 1) (layer "B.Cu") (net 13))
 (segment (start 132.5 85.74) (end 132.5 64.74) (width 1) (layer "B.Cu") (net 13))
 (segment (start 73.8 68.54) (end 73.5 68.24) (width 1) (layer "F.Cu") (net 1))
 (segment (start 81.3 68.54) (end 73.8 68.54) (width 1) (layer "F.Cu") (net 1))
 (via (at 81.3 68.54) (size 2) (drill 0.8) (layers "F.Cu" "B.Cu") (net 1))
 (via (at 73.5 68.24) (size 2) (drill 0.8) (layers "F.Cu" "B.Cu") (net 1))
 (segment (start 49 79.24) (end 60 68.24) (width 1) (layer "B.Cu") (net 1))
 (segment (start 85.64 68.54) (end 81.3 68.54) (width 1) (layer "B.Cu") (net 1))
 (segment (start 49 87.74) (end 49 79.24) (width 1) (layer "B.Cu") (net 1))
 (segment (start 60 68.24) (end 73.5 68.24) (width 1) (layer "B.Cu") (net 1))
 (segment (start 72.25 70.99) (end 81.57 70.99) (width 1) (layer "F.Cu") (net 3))
 (segment (start 81.57 70.99) (end 81.66 71.08) (width 1) (layer "F.Cu") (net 3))
 (via (at 81.66 71.08) (size 2) (drill 0.8) (layers "F.Cu" "B.Cu") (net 3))
 (via (at 72.25 70.99) (size 2) (drill 0.8) (layers "F.Cu" "B.Cu") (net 3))
 (segment (start 72.25 87.99) (end 72.25 70.99) (width 1) (layer "B.Cu") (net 3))
 (segment (start 85.64 71.08) (end 81.66 71.08) (width 1) (layer "B.Cu") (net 3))
 (segment (start 82.25 97.49) (end 82.5 97.24) (width 1) (layer "F.Cu") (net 15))
 (segment (start 72.75 97.49) (end 82.25 97.49) (width 1) (layer "F.Cu") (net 15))
 (via (at 82.5 97.24) (size 2) (drill 0.8) (layers "F.Cu" "B.Cu") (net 15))
 (via (at 72.75 97.49) (size 2) (drill 0.8) (layers "F.Cu" "B.Cu") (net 15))
 (segment (start 84.34 91.4) (end 82.5 93.24) (width 1) (layer "B.Cu") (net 15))
 (segment (start 64.25 97.49) (end 72.75 97.49) (width 1) (layer "B.Cu") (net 15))
 (segment (start 82.5 93.24) (end 82.5 97.24) (width 1) (layer "B.Cu") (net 15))
 (segment (start 85.64 91.4) (end 84.34 91.4) (width 1) (layer "B.Cu") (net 15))
 (segment (start 102.5 92.24) (end 89 105.74) (width 1) (layer "B.Cu") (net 14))
 (segment (start 69 126.24) (end 52 109.24) (width 1) (layer "B.Cu") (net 14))
 (segment (start 52 84.74) (end 57.5 79.24) (width 1) (layer "B.Cu") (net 14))
 (segment (start 89 116.74) (end 79.5 126.24) (width 1) (layer "B.Cu") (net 14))
 (segment (start 52 109.24) (end 52 84.74) (width 1) (layer "B.Cu") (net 14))
 (segment (start 108.5 71.08) (end 105.66 71.08) (width 1) (layer "B.Cu") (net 14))
 (segment (start 102.5 74.24) (end 102.5 92.24) (width 1) (layer "B.Cu") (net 14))
 (segment (start 105.66 71.08) (end 102.5 74.24) (width 1) (layer "B.Cu") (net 14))
 (segment (start 79.5 126.24) (end 69 126.24) (width 1) (layer "B.Cu") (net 14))
 (segment (start 89 105.74) (end 89 116.74) (width 1) (layer "B.Cu") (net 14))
 (segment (start 85.64 111.72) (end 74.52 111.72) (width 1.5) (layer "B.Cu") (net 5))
 (segment (start 74.52 111.72) (end 73 113.24) (width 1.5) (layer "B.Cu") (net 5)))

